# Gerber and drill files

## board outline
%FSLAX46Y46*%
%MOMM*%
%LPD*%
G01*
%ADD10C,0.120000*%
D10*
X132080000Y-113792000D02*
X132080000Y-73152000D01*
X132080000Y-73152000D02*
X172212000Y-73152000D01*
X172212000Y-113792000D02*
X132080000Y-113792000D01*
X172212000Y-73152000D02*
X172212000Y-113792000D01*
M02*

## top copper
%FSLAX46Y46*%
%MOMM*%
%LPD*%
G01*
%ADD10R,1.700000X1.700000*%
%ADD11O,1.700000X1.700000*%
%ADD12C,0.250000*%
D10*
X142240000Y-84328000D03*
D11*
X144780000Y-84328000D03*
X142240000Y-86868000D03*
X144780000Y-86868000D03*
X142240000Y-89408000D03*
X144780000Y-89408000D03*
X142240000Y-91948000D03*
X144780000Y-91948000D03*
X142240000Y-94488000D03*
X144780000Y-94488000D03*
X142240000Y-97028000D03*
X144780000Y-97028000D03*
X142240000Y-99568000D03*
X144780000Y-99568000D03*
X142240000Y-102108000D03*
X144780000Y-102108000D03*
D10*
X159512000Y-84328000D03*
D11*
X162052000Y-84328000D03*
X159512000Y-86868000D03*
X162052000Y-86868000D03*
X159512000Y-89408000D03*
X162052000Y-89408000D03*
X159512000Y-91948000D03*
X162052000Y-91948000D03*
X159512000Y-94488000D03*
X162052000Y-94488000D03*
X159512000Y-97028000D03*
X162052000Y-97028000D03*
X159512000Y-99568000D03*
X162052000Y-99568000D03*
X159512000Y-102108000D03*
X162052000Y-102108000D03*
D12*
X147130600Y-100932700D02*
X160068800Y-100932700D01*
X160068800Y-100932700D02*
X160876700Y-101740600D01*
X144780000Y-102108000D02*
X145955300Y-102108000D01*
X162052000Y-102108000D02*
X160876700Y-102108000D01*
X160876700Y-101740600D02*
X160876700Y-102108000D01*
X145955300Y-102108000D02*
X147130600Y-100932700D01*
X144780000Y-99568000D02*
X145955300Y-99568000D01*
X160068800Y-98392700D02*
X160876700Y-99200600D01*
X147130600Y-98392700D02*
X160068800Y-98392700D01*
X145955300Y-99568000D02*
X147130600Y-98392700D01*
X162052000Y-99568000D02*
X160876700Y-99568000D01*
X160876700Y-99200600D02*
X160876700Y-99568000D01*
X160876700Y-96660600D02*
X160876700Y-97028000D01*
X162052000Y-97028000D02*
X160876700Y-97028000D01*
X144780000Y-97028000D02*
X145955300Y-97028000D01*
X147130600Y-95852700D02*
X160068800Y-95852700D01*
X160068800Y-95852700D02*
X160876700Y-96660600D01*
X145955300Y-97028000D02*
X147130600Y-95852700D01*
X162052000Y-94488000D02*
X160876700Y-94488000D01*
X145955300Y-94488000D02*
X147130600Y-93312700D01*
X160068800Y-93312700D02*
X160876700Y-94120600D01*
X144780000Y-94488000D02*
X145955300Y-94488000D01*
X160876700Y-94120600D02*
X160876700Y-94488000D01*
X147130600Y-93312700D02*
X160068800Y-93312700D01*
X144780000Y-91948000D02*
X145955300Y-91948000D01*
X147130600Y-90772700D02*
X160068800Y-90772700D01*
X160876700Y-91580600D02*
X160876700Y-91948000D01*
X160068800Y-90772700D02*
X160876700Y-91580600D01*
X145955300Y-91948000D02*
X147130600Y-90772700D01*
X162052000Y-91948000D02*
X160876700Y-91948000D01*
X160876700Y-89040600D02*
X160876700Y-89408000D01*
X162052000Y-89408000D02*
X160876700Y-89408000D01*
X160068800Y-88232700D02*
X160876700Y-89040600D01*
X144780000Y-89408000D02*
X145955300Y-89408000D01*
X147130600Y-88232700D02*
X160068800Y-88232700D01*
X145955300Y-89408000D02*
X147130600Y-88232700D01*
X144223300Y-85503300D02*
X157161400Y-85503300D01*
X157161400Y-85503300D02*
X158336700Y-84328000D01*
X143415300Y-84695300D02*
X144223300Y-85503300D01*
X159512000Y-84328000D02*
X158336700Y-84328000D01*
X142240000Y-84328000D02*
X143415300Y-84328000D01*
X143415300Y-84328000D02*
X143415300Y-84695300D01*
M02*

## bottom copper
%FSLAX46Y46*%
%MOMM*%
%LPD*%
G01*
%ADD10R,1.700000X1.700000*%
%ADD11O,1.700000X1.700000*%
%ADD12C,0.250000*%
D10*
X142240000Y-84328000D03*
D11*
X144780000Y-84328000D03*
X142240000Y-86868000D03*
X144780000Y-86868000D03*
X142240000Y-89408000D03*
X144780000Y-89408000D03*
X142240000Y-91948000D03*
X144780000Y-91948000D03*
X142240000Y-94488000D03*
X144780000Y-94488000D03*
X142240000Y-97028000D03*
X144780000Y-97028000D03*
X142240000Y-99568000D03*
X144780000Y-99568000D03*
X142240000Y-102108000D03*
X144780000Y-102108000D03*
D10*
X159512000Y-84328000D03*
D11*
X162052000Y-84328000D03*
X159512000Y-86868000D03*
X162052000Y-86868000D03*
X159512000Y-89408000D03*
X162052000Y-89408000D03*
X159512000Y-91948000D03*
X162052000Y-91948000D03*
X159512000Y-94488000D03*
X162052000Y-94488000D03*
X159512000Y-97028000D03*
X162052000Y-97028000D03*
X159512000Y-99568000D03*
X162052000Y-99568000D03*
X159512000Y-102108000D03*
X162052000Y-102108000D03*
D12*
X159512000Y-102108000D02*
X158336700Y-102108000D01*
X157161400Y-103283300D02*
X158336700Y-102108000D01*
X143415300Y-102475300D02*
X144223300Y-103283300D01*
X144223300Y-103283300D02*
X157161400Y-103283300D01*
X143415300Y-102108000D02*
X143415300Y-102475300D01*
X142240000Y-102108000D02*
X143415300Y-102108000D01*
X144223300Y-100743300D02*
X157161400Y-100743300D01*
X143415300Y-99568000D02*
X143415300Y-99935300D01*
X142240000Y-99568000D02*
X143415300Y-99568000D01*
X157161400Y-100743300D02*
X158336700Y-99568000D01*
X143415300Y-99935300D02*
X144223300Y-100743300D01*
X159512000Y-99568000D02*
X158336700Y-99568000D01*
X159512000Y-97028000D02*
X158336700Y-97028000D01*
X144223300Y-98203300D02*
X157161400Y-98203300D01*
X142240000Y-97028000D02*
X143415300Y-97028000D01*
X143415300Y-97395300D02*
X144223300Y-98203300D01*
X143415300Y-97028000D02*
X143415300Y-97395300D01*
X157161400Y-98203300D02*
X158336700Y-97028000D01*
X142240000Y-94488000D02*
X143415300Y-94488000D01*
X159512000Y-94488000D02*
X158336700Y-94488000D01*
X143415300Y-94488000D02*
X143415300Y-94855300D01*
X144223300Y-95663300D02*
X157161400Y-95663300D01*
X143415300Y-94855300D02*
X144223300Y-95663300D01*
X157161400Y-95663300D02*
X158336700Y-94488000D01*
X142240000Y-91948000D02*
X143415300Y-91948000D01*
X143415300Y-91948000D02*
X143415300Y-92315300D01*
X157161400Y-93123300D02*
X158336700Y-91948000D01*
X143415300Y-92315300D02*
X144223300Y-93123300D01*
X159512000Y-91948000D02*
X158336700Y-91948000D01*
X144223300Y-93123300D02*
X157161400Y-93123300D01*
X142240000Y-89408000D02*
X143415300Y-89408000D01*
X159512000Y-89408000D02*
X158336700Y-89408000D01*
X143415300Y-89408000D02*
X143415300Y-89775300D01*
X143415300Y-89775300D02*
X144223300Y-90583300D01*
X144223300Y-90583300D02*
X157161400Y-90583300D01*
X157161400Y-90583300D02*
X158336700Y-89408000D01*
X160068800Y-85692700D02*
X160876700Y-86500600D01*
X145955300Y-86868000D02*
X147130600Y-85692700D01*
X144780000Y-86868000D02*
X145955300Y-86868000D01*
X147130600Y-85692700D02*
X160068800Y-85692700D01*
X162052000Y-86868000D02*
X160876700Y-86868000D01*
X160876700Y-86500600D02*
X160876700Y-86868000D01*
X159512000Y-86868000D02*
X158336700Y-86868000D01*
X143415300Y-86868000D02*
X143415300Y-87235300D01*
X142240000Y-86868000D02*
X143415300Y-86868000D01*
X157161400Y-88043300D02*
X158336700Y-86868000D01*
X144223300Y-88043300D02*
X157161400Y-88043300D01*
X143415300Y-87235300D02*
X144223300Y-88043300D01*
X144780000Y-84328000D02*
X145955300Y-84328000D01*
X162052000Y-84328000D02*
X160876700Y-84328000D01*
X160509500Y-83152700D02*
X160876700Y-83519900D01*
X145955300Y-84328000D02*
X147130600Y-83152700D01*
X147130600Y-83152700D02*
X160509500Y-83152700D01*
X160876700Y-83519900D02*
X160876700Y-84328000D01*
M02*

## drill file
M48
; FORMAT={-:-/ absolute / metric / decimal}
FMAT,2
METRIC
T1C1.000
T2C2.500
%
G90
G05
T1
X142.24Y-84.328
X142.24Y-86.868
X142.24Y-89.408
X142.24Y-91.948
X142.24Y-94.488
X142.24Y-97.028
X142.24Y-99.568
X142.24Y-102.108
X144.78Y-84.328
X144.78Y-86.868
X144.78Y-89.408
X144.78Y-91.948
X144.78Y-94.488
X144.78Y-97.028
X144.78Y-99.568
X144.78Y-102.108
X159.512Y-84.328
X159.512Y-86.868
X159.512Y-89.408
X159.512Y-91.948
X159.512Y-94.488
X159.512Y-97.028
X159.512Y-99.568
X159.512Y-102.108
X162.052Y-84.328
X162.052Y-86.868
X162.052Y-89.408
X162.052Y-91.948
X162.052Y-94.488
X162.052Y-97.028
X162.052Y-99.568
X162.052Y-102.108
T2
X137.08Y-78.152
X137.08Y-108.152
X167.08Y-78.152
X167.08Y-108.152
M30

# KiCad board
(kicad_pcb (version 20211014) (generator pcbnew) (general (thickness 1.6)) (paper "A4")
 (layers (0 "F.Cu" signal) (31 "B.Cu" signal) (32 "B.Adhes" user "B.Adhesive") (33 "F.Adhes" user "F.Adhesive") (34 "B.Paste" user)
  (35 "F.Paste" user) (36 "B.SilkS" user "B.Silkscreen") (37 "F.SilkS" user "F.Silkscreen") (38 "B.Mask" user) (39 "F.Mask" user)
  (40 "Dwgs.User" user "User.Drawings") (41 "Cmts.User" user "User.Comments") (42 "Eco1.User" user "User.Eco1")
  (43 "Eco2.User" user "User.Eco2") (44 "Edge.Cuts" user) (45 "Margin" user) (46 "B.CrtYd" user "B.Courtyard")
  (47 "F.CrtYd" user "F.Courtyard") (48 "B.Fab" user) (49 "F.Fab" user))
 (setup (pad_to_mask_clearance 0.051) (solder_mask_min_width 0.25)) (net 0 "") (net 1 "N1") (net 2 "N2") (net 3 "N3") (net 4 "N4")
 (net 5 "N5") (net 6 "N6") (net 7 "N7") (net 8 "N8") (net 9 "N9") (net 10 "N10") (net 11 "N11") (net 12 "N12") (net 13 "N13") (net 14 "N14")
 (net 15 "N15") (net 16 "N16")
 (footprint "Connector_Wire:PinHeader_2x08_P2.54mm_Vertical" (layer "F.Cu") (at 142.24 84.328)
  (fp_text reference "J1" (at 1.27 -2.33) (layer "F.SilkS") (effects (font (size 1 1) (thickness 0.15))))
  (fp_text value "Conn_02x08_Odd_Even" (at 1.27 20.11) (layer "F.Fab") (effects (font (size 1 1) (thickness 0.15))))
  (pad "1" thru_hole rect locked (at 0 0) (size 1.7 1.7) (drill 1) (layers *.Cu *.Mask) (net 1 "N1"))
  (pad "2" thru_hole oval locked (at 2.54 0) (size 1.7 1.7) (drill 1) (layers *.Cu *.Mask) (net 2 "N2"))
  (pad "3" thru_hole oval locked (at 0 2.54) (size 1.7 1.7) (drill 1) (layers *.Cu *.Mask) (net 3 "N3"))
  (pad "4" thru_hole oval locked (at 2.54 2.54) (size 1.7 1.7) (drill 1) (layers *.Cu *.Mask) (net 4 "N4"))
  (pad "5" thru_hole oval locked (at 0 5.08) (size 1.7 1.7) (drill 1) (layers *.Cu *.Mask) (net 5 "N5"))
  (pad "6" thru_hole oval locked (at 2.54 5.08) (size 1.7 1.7) (drill 1) (layers *.Cu *.Mask) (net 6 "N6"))
  (pad "7" thru_hole oval locked (at 0 7.62) (size 1.7 1.7) (drill 1) (layers *.Cu *.Mask) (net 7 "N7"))
  (pad "8" thru_hole oval locked (at 2.54 7.62) (size 1.7 1.7) (drill 1) (layers *.Cu *.Mask) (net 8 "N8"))
  (pad "9" thru_hole oval locked (at 0 10.16) (size 1.7 1.7) (drill 1) (layers *.Cu *.Mask) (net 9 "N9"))
  (pad "10" thru_hole oval locked (at 2.54 10.16) (size 1.7 1.7) (drill 1) (layers *.Cu *.Mask) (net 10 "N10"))
  (pad "11" thru_hole oval locked (at 0 12.7) (size 1.7 1.7) (drill 1) (layers *.Cu *.Mask) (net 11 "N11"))
  (pad "12" thru_hole oval locked (at 2.54 12.7) (size 1.7 1.7) (drill 1) (layers *.Cu *.Mask) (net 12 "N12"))
  (pad "13" thru_hole oval locked (at 0 15.24) (size 1.7 1.7) (drill 1) (layers *.Cu *.Mask) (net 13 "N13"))
  (pad "14" thru_hole oval locked (at 2.54 15.24) (size 1.7 1.7) (drill 1) (layers *.Cu *.Mask) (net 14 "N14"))
  (pad "15" thru_hole oval locked (at 0 17.78) (size 1.7 1.7) (drill 1) (layers *.Cu *.Mask) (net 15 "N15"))
  (pad "16" thru_hole oval locked (at 2.54 17.78) (size 1.7 1.7) (drill 1) (layers *.Cu *.Mask) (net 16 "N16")))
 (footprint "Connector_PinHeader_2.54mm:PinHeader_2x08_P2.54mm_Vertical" (layer "F.Cu") (at 159.512 84.328)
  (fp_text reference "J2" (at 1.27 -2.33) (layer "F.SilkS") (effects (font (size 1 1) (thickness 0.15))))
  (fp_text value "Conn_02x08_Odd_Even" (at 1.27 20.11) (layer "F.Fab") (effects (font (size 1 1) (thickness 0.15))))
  (pad "1" thru_hole rect locked (at 0 0) (size 1.7 1.7) (drill 1) (layers *.Cu *.Mask) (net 1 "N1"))
  (pad "2" thru_hole oval locked (at 2.54 0) (size 1.7 1.7) (drill 1) (layers *.Cu *.Mask) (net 2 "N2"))
  (pad "3" thru_hole oval locked (at 0 2.54) (size 1.7 1.7) (drill 1) (layers *.Cu *.Mask) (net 3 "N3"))
  (pad "4" thru_hole oval locked (at 2.54 2.54) (size 1.7 1.7) (drill 1) (layers *.Cu *.Mask) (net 4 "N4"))
  (pad "5" thru_hole oval locked (at 0 5.08) (size 1.7 1.7) (drill 1) (layers *.Cu *.Mask) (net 5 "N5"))
  (pad "6" thru_hole oval locked (at 2.54 5.08) (size 1.7 1.7) (drill 1) (layers *.Cu *.Mask) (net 6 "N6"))
  (pad "7" thru_hole oval locked (at 0 7.62) (size 1.7 1.7) (drill 1) (layers *.Cu *.Mask) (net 7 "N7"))
  (pad "8" thru_hole oval locked (at 2.54 7.62) (size 1.7 1.7) (drill 1) (layers *.Cu *.Mask) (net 8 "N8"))
  (pad "9" thru_hole oval locked (at 0 10.16) (size 1.7 1.7) (drill 1) (layers *.Cu *.Mask) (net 9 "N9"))
  (pad "10" thru_hole oval locked (at 2.54 10.16) (size 1.7 1.7) (drill 1) (layers *.Cu *.Mask) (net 10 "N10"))
  (pad "11" thru_hole oval locked (at 0 12.7) (size 1.7 1.7) (drill 1) (layers *.Cu *.Mask) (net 11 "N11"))
  (pad "12" thru_hole oval locked (at 2.54 12.7) (size 1.7 1.7) (drill 1) (layers *.Cu *.Mask) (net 12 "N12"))
  (pad "13" thru_hole oval locked (at 0 15.24) (size 1.7 1.7) (drill 1) (layers *.Cu *.Mask) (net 13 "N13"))
  (pad "14" thru_hole oval locked (at 2.54 15.24) (size 1.7 1.7) (drill 1) (layers *.Cu *.Mask) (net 14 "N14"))
  (pad "15" thru_hole oval locked (at 0 17.78) (size 1.7 1.7) (drill 1) (layers *.Cu *.Mask) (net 15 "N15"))
  (pad "16" thru_hole oval locked (at 2.54 17.78) (size 1.7 1.7) (drill 1) (layers *.Cu *.Mask) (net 16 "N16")))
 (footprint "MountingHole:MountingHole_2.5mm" (layer "F.Cu") (at 137.08 78.152)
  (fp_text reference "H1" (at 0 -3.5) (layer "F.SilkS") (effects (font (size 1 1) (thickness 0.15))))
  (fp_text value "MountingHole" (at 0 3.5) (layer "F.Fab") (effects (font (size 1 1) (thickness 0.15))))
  (pad "" np_thru_hole circle locked (at 0 0) (size 2.5 2.5) (drill 2.5) (layers *.Cu *.Mask)))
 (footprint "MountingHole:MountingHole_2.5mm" (layer "F.Cu") (at 137.08 108.152)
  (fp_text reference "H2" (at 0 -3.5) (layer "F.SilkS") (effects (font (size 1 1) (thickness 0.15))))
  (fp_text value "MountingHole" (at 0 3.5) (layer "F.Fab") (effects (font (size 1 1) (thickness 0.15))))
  (pad "" np_thru_hole circle locked (at 0 0) (size 2.5 2.5) (drill 2.5) (layers *.Cu *.Mask)))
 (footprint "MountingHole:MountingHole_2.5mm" (layer "F.Cu") (at 167.08 78.152)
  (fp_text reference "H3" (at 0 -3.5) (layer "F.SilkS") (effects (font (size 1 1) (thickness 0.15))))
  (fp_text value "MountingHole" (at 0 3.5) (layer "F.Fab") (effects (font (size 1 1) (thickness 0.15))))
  (pad "" np_thru_hole circle locked (at 0 0) (size 2.5 2.5) (drill 2.5) (layers *.Cu *.Mask)))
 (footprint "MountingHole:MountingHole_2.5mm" (layer "F.Cu") (at 167.08 108.152)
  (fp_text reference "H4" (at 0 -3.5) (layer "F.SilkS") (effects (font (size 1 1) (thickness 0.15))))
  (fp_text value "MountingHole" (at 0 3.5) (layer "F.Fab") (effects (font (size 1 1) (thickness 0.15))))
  (pad "" np_thru_hole circle locked (at 0 0) (size 2.5 2.5) (drill 2.5) (layers *.Cu *.Mask)))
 (gr_line (start 132.08 113.792) (end 132.08 73.152) (layer "Edge.Cuts") (width 0.12))
 (gr_line (start 132.08 73.152) (end 172.212 73.152) (layer "Edge.Cuts") (width 0.12))
 (gr_line (start 172.212 113.792) (end 132.08 113.792) (layer "Edge.Cuts") (width 0.12))
 (gr_line (start 172.212 73.152) (end 172.212 113.792) (layer "Edge.Cuts") (width 0.12))
 (segment (start 147.1306 100.9327) (end 160.0688 100.9327) (width 0.25) (layer "F.Cu") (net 16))
 (segment (start 160.0688 100.9327) (end 160.8767 101.7406) (width 0.25) (layer "F.Cu") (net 16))
 (segment (start 144.78 102.108) (end 145.9553 102.108) (width 0.25) (layer "F.Cu") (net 16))
 (segment (start 162.052 102.108) (end 160.8767 102.108) (width 0.25) (layer "F.Cu") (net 16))
 (segment (start 160.8767 101.7406) (end 160.8767 102.108) (width 0.25) (layer "F.Cu") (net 16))
 (segment (start 145.9553 102.108) (end 147.1306 100.9327) (width 0.25) (layer "F.Cu") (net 16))
 (segment (start 159.512 102.108) (end 158.3367 102.108) (width 0.25) (layer "B.Cu") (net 15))
 (segment (start 157.1614 103.2833) (end 158.3367 102.108) (width 0.25) (layer "B.Cu") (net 15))
 (segment (start 143.4153 102.4753) (end 144.2233 103.2833) (width 0.25) (layer "B.Cu") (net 15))
 (segment (start 144.2233 103.2833) (end 157.1614 103.2833) (width 0.25) (layer "B.Cu") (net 15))
 (segment (start 143.4153 102.108) (end 143.4153 102.4753) (width 0.25) (layer "B.Cu") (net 15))
 (segment (start 142.24 102.108) (end 143.4153 102.108) (width 0.25) (layer "B.Cu") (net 15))
 (segment (start 144.78 99.568) (end 145.9553 99.568) (width 0.25) (layer "F.Cu") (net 14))
 (segment (start 160.0688 98.3927) (end 160.8767 99.2006) (width 0.25) (layer "F.Cu") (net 14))
 (segment (start 147.1306 98.3927) (end 160.0688 98.3927) (width 0.25) (layer "F.Cu") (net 14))
 (segment (start 145.9553 99.568) (end 147.1306 98.3927) (width 0.25) (layer "F.Cu") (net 14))
 (segment (start 162.052 99.568) (end 160.8767 99.568) (width 0.25) (layer "F.Cu") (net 14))
 (segment (start 160.8767 99.2006) (end 160.8767 99.568) (width 0.25) (layer "F.Cu") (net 14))
 (segment (start 144.2233 100.7433) (end 157.1614 100.7433) (width 0.25) (layer "B.Cu") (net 13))
 (segment (start 143.4153 99.568) (end 143.4153 99.9353) (width 0.25) (layer "B.Cu") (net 13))
 (segment (start 142.24 99.568) (end 143.4153 99.568) (width 0.25) (layer "B.Cu") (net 13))
 (segment (start 157.1614 100.7433) (end 158.3367 99.568) (width 0.25) (layer "B.Cu") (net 13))
 (segment (start 143.4153 99.9353) (end 144.2233 100.7433) (width 0.25) (layer "B.Cu") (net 13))
 (segment (start 159.512 99.568) (end 158.3367 99.568) (width 0.25) (layer "B.Cu") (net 13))
 (segment (start 160.8767 96.6606) (end 160.8767 97.028) (width 0.25) (layer "F.Cu") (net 12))
 (segment (start 162.052 97.028) (end 160.8767 97.028) (width 0.25) (layer "F.Cu") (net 12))
 (segment (start 144.78 97.028) (end 145.9553 97.028) (width 0.25) (layer "F.Cu") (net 12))
 (segment (start 147.1306 95.8527) (end 160.0688 95.8527) (width 0.25) (layer "F.Cu") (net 12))
 (segment (start 160.0688 95.8527) (end 160.8767 96.6606) (width 0.25) (layer "F.Cu") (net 12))
 (segment (start 145.9553 97.028) (end 147.1306 95.8527) (width 0.25) (layer "F.Cu") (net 12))
 (segment (start 159.512 97.028) (end 158.3367 97.028) (width 0.25) (layer "B.Cu") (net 11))
 (segment (start 144.2233 98.2033) (end 157.1614 98.2033) (width 0.25) (layer "B.Cu") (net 11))
 (segment (start 142.24 97.028) (end 143.4153 97.028) (width 0.25) (layer "B.Cu") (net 11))
 (segment (start 143.4153 97.3953) (end 144.2233 98.2033) (width 0.25) (layer "B.Cu") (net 11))
 (segment (start 143.4153 97.028) (end 143.4153 97.3953) (width 0.25) (layer "B.Cu") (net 11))
 (segment (start 157.1614 98.2033) (end 158.3367 97.028) (width 0.25) (layer "B.Cu") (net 11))
 (segment (start 162.052 94.488) (end 160.8767 94.488) (width 0.25) (layer "F.Cu") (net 10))
 (segment (start 145.9553 94.488) (end 147.1306 93.3127) (width 0.25) (layer "F.Cu") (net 10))
 (segment (start 160.0688 93.3127) (end 160.8767 94.1206) (width 0.25) (layer "F.Cu") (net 10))
 (segment (start 144.78 94.488) (end 145.9553 94.488) (width 0.25) (layer "F.Cu") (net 10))
 (segment (start 160.8767 94.1206) (end 160.8767 94.488) (width 0.25) (layer "F.Cu") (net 10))
 (segment (start 147.1306 93.3127) (end 160.0688 93.3127) (width 0.25) (layer "F.Cu") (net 10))
 (segment (start 142.24 94.488) (end 143.4153 94.488) (width 0.25) (layer "B.Cu") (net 9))
 (segment (start 159.512 94.488) (end 158.3367 94.488) (width 0.25) (layer "B.Cu") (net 9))
 (segment (start 143.4153 94.488) (end 143.4153 94.8553) (width 0.25) (layer "B.Cu") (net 9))
 (segment (start 144.2233 95.6633) (end 157.1614 95.6633) (width 0.25) (layer "B.Cu") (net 9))
 (segment (start 143.4153 94.8553) (end 144.2233 95.6633) (width 0.25) (layer "B.Cu") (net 9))
 (segment (start 157.1614 95.6633) (end 158.3367 94.488) (width 0.25) (layer "B.Cu") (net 9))
 (segment (start 144.78 91.948) (end 145.9553 91.948) (width 0.25) (layer "F.Cu") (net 8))
 (segment (start 147.1306 90.7727) (end 160.0688 90.7727) (width 0.25) (layer "F.Cu") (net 8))
 (segment (start 160.8767 91.5806) (end 160.8767 91.948) (width 0.25) (layer "F.Cu") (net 8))
 (segment (start 160.0688 90.7727) (end 160.8767 91.5806) (width 0.25) (layer "F.Cu") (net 8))
 (segment (start 145.9553 91.948) (end 147.1306 90.7727) (width 0.25) (layer "F.Cu") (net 8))
 (segment (start 162.052 91.948) (end 160.8767 91.948) (width 0.25) (layer "F.Cu") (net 8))
 (segment (start 142.24 91.948) (end 143.4153 91.948) (width 0.25) (layer "B.Cu") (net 7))
 (segment (start 143.4153 91.948) (end 143.4153 92.3153) (width 0.25) (layer "B.Cu") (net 7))
 (segment (start 157.1614 93.1233) (end 158.3367 91.948) (width 0.25) (layer "B.Cu") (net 7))
 (segment (start 143.4153 92.3153) (end 144.2233 93.1233) (width 0.25) (layer "B.Cu") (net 7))
 (segment (start 159.512 91.948) (end 158.3367 91.948) (width 0.25) (layer "B.Cu") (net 7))
 (segment (start 144.2233 93.1233) (end 157.1614 93.1233) (width 0.25) (layer "B.Cu") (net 7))
 (segment (start 160.8767 89.0406) (end 160.8767 89.408) (width 0.25) (layer "F.Cu") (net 6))
 (segment (start 162.052 89.408) (end 160.8767 89.408) (width 0.25) (layer "F.Cu") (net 6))
 (segment (start 160.0688 88.2327) (end 160.8767 89.0406) (width 0.25) (layer "F.Cu") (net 6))
 (segment (start 144.78 89.408) (end 145.9553 89.408) (width 0.25) (layer "F.Cu") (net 6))
 (segment (start 147.1306 88.2327) (end 160.0688 88.2327) (width 0.25) (layer "F.Cu") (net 6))
 (segment (start 145.9553 89.408) (end 147.1306 88.2327) (width 0.25) (layer "F.Cu") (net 6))
 (segment (start 142.24 89.408) (end 143.4153 89.408) (width 0.25) (layer "B.Cu") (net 5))
 (segment (start 159.512 89.408) (end 158.3367 89.408) (width 0.25) (layer "B.Cu") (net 5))
 (segment (start 143.4153 89.408) (end 143.4153 89.7753) (width 0.25) (layer "B.Cu") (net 5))
 (segment (start 143.4153 89.7753) (end 144.2233 90.5833) (width 0.25) (layer "B.Cu") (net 5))
 (segment (start 144.2233 90.5833) (end 157.1614 90.5833) (width 0.25) (layer "B.Cu") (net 5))
 (segment (start 157.1614 90.5833) (end 158.3367 89.408) (width 0.25) (layer "B.Cu") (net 5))
 (segment (start 160.0688 85.6927) (end 160.8767 86.5006) (width 0.25) (layer "B.Cu") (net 4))
 (segment (start 145.9553 86.868) (end 147.1306 85.6927) (width 0.25) (layer "B.Cu") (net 4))
 (segment (start 144.78 86.868) (end 145.9553 86.868) (width 0.25) (layer "B.Cu") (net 4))
 (segment (start 147.1306 85.6927) (end 160.0688 85.6927) (width 0.25) (layer "B.Cu") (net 4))
 (segment (start 162.052 86.868) (end 160.8767 86.868) (width 0.25) (layer "B.Cu") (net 4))
 (segment (start 160.8767 86.5006) (end 160.8767 86.868) (width 0.25) (layer "B.Cu") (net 4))
 (segment (start 159.512 86.868) (end 158.3367 86.868) (width 0.25) (layer "B.Cu") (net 3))
 (segment (start 143.4153 86.868) (end 143.4153 87.2353) (width 0.25) (layer "B.Cu") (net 3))
 (segment (start 142.24 86.868) (end 143.4153 86.868) (width 0.25) (layer "B.Cu") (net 3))
 (segment (start 157.1614 88.0433) (end 158.3367 86.868) (width 0.25) (layer "B.Cu") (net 3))
 (segment (start 144.2233 88.0433) (end 157.1614 88.0433) (width 0.25) (layer "B.Cu") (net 3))
 (segment (start 143.4153 87.2353) (end 144.2233 88.0433) (width 0.25) (layer "B.Cu") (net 3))
 (segment (start 144.78 84.328) (end 145.9553 84.328) (width 0.25) (layer "B.Cu") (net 2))
 (segment (start 162.052 84.328) (end 160.8767 84.328) (width 0.25) (layer "B.Cu") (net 2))
 (segment (start 160.5095 83.1527) (end 160.8767 83.5199) (width 0.25) (layer "B.Cu") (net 2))
 (segment (start 145.9553 84.328) (end 147.1306 83.1527) (width 0.25) (layer "B.Cu") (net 2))
 (segment (start 147.1306 83.1527) (end 160.5095 83.1527) (width 0.25) (layer "B.Cu") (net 2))
 (segment (start 160.8767 83.5199) (end 160.8767 84.328) (width 0.25) (layer "B.Cu") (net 2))
 (segment (start 144.2233 85.5033) (end 157.1614 85.5033) (width 0.25) (layer "F.Cu") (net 1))
 (segment (start 157.1614 85.5033) (end 158.3367 84.328) (width 0.25) (layer "F.Cu") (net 1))
 (segment (start 143.4153 84.6953) (end 144.2233 85.5033) (width 0.25) (layer "F.Cu") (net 1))
 (segment (start 159.512 84.328) (end 158.3367 84.328) (width 0.25) (layer "F.Cu") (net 1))
 (segment (start 142.24 84.328) (end 143.4153 84.328) (width 0.25) (layer "F.Cu") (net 1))
 (segment (start 143.4153 84.328) (end 143.4153 84.6953) (width 0.25) (layer "F.Cu") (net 1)))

